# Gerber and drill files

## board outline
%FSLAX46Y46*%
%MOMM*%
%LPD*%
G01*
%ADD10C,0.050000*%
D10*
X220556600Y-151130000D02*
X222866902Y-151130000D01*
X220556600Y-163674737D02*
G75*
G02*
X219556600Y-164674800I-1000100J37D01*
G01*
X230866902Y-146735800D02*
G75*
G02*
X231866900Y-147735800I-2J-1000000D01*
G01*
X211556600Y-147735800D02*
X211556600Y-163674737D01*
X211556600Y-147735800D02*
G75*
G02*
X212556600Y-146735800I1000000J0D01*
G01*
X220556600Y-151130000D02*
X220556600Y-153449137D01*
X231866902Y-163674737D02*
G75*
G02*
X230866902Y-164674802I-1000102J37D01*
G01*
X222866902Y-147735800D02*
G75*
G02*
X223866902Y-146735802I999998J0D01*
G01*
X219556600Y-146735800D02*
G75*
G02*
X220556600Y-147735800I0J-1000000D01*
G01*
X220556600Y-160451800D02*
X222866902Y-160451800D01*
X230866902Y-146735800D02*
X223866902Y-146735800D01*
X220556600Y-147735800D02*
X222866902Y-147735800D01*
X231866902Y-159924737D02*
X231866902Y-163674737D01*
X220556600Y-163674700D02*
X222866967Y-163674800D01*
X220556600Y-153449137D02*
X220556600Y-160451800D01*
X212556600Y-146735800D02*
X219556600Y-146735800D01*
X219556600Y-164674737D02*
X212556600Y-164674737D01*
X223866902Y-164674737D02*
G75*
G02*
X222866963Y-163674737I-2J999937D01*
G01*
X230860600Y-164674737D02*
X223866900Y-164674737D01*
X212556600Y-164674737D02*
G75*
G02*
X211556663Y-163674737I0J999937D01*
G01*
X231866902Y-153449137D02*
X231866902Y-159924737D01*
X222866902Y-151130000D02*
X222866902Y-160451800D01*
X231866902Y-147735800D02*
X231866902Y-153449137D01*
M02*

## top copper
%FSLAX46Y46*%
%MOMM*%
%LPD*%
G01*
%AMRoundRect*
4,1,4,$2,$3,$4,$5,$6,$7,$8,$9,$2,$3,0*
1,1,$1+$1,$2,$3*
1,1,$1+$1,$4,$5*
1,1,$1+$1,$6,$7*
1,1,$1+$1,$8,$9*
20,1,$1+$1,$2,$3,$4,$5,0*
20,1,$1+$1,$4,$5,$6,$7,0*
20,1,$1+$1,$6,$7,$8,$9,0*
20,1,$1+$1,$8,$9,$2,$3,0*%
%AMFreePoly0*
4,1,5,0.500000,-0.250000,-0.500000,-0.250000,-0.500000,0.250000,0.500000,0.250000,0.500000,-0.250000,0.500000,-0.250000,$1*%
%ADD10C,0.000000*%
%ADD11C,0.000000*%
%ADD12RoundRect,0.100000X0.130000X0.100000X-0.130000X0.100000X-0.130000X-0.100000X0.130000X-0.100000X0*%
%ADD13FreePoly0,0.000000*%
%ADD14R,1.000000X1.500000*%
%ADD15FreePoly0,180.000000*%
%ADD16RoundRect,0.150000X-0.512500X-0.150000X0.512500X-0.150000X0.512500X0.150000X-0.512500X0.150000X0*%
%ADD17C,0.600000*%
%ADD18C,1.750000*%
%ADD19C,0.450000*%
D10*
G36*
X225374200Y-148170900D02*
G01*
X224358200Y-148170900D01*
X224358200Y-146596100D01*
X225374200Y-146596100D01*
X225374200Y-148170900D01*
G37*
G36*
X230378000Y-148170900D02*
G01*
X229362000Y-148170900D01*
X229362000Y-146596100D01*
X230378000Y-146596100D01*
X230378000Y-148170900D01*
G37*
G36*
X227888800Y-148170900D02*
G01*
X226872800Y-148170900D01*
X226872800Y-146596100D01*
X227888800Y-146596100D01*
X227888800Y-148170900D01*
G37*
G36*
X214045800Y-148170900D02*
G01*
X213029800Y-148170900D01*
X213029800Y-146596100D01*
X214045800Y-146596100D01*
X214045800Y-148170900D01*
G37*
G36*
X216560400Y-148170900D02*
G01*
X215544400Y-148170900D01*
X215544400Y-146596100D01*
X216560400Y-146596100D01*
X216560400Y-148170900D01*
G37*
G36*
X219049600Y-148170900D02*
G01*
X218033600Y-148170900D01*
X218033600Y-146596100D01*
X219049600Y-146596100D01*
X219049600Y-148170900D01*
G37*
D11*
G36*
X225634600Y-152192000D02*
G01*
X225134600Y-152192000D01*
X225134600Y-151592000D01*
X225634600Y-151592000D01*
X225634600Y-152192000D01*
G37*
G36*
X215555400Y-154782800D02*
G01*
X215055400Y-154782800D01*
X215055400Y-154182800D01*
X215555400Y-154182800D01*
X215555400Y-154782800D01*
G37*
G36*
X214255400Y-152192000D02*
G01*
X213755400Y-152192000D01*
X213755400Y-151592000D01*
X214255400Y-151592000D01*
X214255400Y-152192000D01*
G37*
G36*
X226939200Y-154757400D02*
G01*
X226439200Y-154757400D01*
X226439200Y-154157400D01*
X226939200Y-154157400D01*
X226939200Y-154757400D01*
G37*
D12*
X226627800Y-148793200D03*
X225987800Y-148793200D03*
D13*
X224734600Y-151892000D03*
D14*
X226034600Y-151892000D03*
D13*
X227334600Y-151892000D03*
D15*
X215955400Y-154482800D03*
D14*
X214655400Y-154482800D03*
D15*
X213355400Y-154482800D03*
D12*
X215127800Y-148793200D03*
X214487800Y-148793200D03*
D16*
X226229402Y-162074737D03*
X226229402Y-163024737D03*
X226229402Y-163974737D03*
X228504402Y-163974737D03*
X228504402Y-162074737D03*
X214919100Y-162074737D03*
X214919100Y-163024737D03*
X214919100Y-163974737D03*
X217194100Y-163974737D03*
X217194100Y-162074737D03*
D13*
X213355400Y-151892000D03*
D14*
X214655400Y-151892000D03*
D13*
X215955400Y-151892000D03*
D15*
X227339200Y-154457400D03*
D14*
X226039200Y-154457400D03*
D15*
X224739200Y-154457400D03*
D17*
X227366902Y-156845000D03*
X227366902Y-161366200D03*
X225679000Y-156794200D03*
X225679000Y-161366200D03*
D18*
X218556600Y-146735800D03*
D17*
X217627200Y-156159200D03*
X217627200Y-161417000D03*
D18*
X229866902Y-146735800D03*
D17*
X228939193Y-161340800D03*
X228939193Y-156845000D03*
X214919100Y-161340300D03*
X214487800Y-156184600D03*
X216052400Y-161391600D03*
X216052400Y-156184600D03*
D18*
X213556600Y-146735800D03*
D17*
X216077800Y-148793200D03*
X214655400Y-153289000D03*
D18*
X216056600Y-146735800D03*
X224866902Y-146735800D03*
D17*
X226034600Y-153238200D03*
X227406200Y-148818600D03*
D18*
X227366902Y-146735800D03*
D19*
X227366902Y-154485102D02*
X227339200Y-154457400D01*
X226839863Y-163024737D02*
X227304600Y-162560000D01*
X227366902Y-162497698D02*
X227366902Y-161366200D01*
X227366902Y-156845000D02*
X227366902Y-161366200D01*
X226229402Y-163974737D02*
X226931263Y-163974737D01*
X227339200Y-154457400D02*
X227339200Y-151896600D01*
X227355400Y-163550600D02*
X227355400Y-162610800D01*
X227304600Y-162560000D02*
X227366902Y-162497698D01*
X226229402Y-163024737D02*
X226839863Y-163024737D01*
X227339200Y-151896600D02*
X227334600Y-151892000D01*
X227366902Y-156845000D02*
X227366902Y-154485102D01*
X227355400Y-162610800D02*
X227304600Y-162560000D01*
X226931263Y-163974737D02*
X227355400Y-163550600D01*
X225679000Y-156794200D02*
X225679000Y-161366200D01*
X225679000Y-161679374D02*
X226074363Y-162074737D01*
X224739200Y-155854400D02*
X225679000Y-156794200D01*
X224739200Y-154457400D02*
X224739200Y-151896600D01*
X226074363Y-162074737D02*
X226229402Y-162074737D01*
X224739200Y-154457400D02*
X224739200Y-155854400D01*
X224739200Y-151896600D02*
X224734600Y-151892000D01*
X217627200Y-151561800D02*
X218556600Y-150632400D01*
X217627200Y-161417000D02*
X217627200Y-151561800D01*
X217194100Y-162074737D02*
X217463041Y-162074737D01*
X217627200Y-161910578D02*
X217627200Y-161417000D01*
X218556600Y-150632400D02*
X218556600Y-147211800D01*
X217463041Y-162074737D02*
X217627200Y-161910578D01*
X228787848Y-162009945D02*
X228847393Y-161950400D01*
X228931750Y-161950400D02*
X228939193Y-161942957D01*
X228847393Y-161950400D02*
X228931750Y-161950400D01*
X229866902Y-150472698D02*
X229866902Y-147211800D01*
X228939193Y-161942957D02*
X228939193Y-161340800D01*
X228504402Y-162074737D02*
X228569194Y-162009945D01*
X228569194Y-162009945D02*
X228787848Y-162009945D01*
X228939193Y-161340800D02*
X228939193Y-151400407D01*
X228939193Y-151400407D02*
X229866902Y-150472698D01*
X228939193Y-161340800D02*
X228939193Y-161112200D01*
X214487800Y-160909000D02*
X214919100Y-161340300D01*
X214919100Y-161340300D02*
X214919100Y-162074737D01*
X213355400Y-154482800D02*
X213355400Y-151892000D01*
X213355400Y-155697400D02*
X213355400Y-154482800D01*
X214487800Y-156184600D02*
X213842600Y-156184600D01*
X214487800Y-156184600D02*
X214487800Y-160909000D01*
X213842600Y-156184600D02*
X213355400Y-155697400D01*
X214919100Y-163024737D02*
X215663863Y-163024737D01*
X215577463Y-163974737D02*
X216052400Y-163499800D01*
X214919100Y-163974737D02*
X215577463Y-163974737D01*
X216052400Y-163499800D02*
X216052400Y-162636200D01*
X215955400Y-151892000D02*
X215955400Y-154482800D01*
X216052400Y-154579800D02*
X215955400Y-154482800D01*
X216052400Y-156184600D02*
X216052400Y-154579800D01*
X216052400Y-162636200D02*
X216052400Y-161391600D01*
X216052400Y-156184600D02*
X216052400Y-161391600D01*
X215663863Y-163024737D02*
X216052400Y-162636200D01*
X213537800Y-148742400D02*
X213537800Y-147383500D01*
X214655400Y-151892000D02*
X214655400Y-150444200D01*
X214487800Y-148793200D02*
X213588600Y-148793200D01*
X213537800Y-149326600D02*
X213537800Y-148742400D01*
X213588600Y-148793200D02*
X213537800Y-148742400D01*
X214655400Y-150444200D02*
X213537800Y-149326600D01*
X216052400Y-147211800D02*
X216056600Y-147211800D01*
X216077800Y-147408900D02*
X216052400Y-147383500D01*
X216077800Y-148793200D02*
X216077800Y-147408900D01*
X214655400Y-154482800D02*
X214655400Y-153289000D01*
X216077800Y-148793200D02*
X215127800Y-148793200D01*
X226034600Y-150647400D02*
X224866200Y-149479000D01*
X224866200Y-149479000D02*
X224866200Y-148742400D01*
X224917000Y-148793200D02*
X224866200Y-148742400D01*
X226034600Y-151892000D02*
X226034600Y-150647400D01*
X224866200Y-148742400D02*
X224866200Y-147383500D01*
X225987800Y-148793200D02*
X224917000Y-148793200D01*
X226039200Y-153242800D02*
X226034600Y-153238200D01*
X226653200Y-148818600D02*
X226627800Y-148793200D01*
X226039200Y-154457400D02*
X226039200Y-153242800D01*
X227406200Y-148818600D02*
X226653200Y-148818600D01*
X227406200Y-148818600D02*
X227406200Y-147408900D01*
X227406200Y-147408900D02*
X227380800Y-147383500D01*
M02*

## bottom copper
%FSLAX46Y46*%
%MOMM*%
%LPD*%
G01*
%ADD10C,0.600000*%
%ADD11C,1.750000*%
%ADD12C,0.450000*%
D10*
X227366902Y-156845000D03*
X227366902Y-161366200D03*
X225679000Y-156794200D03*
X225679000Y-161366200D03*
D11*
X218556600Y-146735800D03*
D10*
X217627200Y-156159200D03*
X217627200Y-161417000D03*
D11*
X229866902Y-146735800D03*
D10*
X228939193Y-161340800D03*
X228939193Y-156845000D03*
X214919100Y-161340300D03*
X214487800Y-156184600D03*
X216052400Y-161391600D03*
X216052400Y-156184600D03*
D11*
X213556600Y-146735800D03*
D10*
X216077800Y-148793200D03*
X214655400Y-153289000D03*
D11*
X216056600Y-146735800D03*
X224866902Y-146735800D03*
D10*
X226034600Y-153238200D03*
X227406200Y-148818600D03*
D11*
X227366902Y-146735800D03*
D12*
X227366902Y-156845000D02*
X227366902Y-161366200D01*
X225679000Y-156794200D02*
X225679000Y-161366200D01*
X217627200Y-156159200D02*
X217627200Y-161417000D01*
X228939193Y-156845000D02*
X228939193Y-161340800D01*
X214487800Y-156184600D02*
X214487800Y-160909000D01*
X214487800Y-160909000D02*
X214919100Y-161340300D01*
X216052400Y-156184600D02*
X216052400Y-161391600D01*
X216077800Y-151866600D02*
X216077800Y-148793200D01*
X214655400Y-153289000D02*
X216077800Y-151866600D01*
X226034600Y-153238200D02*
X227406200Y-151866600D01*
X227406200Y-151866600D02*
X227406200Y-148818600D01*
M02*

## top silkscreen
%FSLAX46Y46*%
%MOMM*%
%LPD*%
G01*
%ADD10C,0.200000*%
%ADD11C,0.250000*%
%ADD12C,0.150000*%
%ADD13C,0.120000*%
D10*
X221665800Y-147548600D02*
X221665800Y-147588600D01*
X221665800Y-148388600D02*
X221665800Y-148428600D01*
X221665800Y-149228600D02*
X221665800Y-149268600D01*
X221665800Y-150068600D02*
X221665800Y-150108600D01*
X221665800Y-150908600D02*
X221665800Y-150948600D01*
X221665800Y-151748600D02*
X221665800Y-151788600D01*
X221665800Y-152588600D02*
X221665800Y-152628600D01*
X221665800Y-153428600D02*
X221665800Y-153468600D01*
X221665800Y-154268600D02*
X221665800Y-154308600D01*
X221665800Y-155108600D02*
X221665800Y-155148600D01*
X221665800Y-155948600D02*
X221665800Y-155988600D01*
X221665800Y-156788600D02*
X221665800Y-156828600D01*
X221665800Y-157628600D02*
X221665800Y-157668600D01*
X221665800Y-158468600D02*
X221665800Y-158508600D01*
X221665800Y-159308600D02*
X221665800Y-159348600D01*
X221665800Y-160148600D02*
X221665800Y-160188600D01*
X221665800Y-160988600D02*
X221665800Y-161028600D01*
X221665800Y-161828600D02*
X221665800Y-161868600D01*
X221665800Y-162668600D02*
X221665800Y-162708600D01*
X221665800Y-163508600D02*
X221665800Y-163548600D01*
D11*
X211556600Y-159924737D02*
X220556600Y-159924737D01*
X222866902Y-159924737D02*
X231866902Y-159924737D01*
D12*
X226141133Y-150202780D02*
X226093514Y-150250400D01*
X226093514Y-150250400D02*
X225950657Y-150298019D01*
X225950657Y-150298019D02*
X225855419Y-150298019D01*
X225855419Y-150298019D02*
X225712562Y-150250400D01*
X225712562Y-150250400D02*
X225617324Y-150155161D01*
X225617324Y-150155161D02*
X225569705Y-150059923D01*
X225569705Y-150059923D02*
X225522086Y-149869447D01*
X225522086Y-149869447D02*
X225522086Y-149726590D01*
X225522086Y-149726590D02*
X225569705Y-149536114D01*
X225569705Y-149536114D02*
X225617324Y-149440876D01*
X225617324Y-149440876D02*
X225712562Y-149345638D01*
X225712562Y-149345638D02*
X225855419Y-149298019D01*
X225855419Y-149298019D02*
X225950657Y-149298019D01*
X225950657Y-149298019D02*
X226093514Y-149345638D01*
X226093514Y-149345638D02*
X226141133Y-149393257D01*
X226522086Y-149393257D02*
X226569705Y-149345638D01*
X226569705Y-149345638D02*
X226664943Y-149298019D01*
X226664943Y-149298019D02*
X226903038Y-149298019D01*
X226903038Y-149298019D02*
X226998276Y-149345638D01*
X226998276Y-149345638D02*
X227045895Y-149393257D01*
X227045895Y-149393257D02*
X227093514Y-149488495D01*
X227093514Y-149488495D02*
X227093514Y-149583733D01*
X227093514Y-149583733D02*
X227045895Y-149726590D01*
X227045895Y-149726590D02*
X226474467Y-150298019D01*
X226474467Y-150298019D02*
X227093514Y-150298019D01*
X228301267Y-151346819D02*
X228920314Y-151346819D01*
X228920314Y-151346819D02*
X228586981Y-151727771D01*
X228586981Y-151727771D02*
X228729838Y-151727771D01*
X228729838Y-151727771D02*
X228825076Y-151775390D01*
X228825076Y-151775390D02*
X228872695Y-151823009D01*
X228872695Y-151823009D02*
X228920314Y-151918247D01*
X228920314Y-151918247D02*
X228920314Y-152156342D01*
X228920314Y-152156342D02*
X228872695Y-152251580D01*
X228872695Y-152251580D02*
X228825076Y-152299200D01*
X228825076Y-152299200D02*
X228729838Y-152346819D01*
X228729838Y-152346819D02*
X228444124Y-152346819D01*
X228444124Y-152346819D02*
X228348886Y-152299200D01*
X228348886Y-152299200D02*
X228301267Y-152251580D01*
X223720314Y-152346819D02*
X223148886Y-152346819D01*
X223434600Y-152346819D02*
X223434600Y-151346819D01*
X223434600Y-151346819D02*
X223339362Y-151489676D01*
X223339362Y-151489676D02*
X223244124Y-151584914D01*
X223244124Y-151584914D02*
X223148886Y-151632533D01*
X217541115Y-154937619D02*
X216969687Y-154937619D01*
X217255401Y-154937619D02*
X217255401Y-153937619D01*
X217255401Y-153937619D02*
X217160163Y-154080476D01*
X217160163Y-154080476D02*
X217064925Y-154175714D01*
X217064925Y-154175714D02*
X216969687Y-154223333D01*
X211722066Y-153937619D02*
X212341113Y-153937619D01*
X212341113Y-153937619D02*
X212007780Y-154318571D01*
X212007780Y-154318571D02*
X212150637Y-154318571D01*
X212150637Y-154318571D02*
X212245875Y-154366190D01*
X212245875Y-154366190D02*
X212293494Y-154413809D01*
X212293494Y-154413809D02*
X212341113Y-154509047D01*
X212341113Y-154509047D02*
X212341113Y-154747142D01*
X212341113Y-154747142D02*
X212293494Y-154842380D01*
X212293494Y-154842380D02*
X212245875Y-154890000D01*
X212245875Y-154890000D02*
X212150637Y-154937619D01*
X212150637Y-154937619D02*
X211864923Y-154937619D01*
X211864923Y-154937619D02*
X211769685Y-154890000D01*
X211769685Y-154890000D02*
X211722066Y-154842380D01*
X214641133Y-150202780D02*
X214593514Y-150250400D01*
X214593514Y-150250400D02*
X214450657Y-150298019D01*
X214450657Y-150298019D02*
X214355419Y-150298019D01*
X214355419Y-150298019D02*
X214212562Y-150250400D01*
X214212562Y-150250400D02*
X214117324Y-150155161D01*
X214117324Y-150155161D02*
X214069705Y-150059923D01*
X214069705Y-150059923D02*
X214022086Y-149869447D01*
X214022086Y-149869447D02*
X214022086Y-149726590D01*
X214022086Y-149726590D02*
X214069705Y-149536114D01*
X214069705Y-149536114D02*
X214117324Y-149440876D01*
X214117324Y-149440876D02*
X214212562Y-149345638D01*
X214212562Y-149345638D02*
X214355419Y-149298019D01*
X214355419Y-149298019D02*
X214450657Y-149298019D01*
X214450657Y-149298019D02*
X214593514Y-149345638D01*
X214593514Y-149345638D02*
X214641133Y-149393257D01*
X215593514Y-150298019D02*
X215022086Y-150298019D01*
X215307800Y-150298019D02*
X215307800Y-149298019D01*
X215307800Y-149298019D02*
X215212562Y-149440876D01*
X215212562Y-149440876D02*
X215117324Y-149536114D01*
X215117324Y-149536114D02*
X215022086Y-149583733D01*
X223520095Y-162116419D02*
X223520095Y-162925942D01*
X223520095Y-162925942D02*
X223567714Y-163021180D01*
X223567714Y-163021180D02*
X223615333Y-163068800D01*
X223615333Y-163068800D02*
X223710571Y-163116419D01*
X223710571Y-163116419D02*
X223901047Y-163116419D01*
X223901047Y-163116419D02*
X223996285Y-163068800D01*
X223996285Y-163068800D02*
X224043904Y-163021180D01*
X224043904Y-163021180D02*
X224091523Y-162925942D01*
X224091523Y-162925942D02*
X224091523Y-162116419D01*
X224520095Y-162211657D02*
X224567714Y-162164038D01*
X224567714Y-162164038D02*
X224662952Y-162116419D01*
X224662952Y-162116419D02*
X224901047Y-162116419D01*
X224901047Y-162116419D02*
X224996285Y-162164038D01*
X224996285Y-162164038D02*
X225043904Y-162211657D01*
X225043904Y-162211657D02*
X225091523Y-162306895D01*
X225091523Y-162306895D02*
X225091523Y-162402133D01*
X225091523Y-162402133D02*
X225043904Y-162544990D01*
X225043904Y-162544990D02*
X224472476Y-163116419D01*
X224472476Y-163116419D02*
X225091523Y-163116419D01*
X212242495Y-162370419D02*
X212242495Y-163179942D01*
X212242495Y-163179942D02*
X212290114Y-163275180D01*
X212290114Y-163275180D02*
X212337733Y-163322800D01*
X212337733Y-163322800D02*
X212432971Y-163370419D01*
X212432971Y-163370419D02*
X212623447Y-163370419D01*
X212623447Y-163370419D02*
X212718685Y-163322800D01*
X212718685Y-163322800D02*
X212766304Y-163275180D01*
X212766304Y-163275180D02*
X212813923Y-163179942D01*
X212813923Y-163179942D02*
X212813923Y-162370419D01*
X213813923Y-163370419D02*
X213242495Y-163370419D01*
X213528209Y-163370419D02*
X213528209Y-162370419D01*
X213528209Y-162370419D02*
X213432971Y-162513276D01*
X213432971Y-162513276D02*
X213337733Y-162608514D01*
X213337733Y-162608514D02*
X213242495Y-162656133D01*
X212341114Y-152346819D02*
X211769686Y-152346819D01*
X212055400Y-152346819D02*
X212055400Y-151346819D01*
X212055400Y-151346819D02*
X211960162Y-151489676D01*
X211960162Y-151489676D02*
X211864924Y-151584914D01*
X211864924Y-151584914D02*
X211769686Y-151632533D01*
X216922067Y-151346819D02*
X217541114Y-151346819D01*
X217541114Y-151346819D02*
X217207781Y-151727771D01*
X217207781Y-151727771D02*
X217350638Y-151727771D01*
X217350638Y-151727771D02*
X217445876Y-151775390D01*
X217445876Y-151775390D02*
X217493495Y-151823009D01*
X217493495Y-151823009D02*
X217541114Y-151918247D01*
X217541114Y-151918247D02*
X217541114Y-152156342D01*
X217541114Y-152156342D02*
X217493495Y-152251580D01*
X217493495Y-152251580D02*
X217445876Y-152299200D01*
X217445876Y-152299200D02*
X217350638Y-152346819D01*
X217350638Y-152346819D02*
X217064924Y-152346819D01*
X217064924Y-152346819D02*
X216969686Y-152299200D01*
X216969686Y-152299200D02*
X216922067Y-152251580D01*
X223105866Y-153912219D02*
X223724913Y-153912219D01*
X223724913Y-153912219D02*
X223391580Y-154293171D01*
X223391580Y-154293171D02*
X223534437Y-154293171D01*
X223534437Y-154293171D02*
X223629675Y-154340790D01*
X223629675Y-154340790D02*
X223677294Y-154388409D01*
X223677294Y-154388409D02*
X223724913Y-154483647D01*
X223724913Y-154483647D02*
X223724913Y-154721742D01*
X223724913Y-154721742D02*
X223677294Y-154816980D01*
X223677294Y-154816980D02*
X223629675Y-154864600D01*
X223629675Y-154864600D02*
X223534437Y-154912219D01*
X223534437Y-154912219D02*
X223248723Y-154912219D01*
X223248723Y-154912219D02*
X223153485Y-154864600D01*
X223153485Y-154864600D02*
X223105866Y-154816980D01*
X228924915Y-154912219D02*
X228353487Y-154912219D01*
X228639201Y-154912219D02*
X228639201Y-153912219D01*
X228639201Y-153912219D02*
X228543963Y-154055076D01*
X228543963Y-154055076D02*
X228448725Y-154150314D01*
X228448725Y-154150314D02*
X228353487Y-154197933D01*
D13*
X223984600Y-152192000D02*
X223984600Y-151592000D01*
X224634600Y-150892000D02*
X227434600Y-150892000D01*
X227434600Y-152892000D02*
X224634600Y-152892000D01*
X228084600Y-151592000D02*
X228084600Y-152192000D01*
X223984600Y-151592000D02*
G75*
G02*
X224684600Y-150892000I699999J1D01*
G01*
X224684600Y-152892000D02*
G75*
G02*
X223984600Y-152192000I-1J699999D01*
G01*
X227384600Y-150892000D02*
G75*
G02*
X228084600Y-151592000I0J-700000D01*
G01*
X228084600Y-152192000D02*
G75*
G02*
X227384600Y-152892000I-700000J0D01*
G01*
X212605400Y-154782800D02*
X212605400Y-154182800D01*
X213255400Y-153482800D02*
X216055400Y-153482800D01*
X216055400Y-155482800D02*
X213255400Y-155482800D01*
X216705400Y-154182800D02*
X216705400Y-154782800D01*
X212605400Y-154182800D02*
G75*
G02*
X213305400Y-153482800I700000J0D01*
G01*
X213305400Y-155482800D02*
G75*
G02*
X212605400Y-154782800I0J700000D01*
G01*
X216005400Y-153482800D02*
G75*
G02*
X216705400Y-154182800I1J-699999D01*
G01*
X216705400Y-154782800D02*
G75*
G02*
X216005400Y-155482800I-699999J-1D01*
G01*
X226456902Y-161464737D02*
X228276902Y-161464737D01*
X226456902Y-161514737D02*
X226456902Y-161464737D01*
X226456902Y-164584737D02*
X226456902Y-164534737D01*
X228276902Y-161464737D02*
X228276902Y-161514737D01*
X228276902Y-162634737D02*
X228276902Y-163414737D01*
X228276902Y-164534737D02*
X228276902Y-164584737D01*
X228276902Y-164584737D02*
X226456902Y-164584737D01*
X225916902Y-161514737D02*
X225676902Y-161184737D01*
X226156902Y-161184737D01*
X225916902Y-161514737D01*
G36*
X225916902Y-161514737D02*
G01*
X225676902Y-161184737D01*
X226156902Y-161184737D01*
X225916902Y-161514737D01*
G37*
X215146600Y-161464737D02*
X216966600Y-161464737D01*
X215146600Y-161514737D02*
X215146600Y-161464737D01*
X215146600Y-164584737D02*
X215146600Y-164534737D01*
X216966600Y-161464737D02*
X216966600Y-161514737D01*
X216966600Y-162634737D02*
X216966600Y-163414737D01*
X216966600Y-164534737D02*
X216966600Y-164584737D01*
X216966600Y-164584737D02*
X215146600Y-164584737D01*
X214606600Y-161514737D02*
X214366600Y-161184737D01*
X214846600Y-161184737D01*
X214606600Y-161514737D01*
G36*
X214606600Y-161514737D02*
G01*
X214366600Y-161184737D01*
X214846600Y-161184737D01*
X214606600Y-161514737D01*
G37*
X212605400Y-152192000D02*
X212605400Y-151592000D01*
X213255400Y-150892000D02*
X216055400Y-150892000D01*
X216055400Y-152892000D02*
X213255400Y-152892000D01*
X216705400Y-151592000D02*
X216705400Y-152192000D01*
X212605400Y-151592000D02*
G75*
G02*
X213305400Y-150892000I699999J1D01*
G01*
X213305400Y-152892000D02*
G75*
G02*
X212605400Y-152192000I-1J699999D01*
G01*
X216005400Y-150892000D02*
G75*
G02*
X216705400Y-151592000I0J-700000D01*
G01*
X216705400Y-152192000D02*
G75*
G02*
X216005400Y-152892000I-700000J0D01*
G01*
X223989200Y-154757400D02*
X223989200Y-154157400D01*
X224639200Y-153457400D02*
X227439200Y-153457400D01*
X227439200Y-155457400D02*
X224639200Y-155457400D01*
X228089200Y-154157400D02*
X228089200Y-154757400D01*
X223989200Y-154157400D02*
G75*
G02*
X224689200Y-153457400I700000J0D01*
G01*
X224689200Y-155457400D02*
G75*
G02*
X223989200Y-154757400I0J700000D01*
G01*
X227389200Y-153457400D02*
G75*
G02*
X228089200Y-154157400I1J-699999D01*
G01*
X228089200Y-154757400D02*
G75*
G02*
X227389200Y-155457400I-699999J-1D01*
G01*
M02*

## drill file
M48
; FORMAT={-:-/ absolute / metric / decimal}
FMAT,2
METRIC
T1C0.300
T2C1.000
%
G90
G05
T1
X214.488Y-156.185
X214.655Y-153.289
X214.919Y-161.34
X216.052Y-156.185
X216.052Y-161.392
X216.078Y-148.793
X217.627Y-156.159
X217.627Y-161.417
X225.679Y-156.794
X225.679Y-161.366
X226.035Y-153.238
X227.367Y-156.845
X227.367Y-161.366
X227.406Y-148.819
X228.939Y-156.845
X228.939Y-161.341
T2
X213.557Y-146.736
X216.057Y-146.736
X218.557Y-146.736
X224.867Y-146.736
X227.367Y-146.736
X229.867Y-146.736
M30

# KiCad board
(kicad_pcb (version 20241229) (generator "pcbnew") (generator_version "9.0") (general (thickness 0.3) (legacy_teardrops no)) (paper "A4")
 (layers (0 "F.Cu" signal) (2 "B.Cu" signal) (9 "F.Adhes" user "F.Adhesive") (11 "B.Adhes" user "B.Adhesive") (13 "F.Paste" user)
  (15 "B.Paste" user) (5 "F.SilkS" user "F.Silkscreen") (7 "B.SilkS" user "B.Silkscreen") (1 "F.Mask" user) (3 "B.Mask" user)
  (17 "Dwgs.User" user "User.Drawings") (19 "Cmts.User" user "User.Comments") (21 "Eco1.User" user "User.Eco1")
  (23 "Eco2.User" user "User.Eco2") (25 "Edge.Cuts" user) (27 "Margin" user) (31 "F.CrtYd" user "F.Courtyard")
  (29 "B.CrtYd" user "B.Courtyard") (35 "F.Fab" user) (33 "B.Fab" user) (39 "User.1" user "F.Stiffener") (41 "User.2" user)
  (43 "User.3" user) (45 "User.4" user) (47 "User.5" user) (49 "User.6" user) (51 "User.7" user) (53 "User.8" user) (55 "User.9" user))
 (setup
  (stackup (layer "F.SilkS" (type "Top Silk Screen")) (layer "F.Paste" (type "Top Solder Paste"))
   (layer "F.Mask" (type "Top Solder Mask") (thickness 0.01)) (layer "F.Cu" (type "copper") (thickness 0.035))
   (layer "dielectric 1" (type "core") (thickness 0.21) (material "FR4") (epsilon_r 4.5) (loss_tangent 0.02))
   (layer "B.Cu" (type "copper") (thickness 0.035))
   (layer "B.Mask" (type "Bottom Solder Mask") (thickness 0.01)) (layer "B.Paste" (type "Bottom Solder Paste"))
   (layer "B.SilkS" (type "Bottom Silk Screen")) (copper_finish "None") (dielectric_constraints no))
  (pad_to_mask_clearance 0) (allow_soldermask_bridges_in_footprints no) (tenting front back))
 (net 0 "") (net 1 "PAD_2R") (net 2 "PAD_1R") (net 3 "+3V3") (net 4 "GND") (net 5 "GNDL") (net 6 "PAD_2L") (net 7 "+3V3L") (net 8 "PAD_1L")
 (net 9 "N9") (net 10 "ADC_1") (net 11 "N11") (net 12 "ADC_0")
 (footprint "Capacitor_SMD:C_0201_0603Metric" (layer "F.Cu") (at 226.3078 148.7932 180)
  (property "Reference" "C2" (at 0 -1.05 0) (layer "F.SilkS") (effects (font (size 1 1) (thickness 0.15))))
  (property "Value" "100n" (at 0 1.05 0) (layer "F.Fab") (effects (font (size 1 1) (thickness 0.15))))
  (pad "" smd roundrect (at -0.345 0 180) (size 0.318 0.36) (layers "F.Paste") (roundrect_rratio 0.25))
  (pad "" smd roundrect (at 0.345 0 180) (size 0.318 0.36) (layers "F.Paste") (roundrect_rratio 0.25))
  (pad "1" smd roundrect (at -0.32 0 180) (size 0.46 0.4) (layers "F.Cu" "F.Mask") (roundrect_rratio 0.25) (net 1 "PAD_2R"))
  (pad "2" smd roundrect (at 0.32 0 180) (size 0.46 0.4) (layers "F.Cu" "F.Mask") (roundrect_rratio 0.25) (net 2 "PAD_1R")))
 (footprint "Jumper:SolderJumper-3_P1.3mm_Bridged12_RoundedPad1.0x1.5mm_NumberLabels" (layer "F.Cu") (at 226.0346 151.892)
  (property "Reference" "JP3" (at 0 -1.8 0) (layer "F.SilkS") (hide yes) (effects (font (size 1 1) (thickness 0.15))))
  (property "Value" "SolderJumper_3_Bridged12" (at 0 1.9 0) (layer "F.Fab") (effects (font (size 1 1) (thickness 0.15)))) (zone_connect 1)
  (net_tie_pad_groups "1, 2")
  (fp_poly (pts (xy -0.9 -0.3) (xy -0.4 -0.3) (xy -0.4 0.3) (xy -0.9 0.3)) (stroke (width 0) (type solid)) (fill yes) (layer "F.Cu"))
  (fp_line (start -2.05 0.3) (end -2.05 -0.3) (stroke (width 0.12) (type solid)) (layer "F.SilkS"))
  (fp_line (start -1.4 -1) (end 1.4 -1) (stroke (width 0.12) (type solid)) (layer "F.SilkS"))
  (fp_line (start 1.4 1) (end -1.4 1) (stroke (width 0.12) (type solid)) (layer "F.SilkS"))
  (fp_line (start 2.05 -0.3) (end 2.05 0.3) (stroke (width 0.12) (type solid)) (layer "F.SilkS"))
  (fp_arc (start -2.05 -0.3) (mid -1.844975 -0.794975) (end -1.35 -1) (stroke (width 0.12) (type solid)) (layer "F.SilkS"))
  (fp_arc (start -1.35 1) (mid -1.844975 0.794975) (end -2.05 0.3) (stroke (width 0.12) (type solid)) (layer "F.SilkS"))
  (fp_arc (start 1.35 -1) (mid 1.844975 -0.794975) (end 2.05 -0.3) (stroke (width 0.12) (type solid)) (layer "F.SilkS"))
  (fp_arc (start 2.05 0.3) (mid 1.844975 0.794975) (end 1.35 1) (stroke (width 0.12) (type solid)) (layer "F.SilkS"))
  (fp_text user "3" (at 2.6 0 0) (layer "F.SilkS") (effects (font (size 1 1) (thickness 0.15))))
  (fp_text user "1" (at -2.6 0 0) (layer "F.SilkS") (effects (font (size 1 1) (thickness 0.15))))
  (pad "1" smd custom (at -1.3 0) (size 1 0.5) (layers "F.Cu" "F.Mask") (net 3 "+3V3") (zone_connect 2) (thermal_bridge_angle 45)
   (options (clearance outline) (anchor rect)) (primitives))
  (pad "2" smd rect (at 0 0) (size 1 1.5) (layers "F.Cu" "F.Mask") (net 2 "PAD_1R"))
  (pad "3" smd custom (at 1.3 0) (size 1 0.5) (layers "F.Cu" "F.Mask") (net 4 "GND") (zone_connect 2) (thermal_bridge_angle 45)
   (options (clearance outline) (anchor rect)) (primitives)))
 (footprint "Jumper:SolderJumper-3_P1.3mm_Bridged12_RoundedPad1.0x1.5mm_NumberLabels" (layer "F.Cu") (at 214.6554 154.4828 180)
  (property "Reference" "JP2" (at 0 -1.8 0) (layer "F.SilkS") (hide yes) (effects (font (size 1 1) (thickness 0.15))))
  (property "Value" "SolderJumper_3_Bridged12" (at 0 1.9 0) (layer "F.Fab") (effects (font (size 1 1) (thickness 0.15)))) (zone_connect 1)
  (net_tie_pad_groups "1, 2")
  (fp_poly (pts (xy -0.9 -0.3) (xy -0.4 -0.3) (xy -0.4 0.3) (xy -0.9 0.3)) (stroke (width 0) (type solid)) (fill yes) (layer "F.Cu"))
  (fp_line (start 2.05 -0.3) (end 2.05 0.3) (stroke (width 0.12) (type solid)) (layer "F.SilkS"))
  (fp_line (start 1.4 1) (end -1.4 1) (stroke (width 0.12) (type solid)) (layer "F.SilkS"))
  (fp_line (start -1.4 -1) (end 1.4 -1) (stroke (width 0.12) (type solid)) (layer "F.SilkS"))
  (fp_line (start -2.05 0.3) (end -2.05 -0.3) (stroke (width 0.12) (type solid)) (layer "F.SilkS"))
  (fp_arc (start 2.05 0.3) (mid 1.844975 0.794975) (end 1.35 1) (stroke (width 0.12) (type solid)) (layer "F.SilkS"))
  (fp_arc (start 1.35 -1) (mid 1.844975 -0.794975) (end 2.05 -0.3) (stroke (width 0.12) (type solid)) (layer "F.SilkS"))
  (fp_arc (start -1.35 1) (mid -1.844975 0.794975) (end -2.05 0.3) (stroke (width 0.12) (type solid)) (layer "F.SilkS"))
  (fp_arc (start -2.05 -0.3) (mid -1.844975 -0.794975) (end -1.35 -1) (stroke (width 0.12) (type solid)) (layer "F.SilkS"))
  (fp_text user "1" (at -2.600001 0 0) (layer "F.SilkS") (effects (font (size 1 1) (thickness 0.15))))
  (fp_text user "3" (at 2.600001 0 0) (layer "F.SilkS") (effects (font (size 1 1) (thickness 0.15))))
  (pad "1" smd custom (at -1.3 0 180) (size 1 0.5) (layers "F.Cu" "F.Mask") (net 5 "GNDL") (zone_connect 2) (thermal_bridge_angle 45)
   (options (clearance outline) (anchor rect)) (primitives))
  (pad "2" smd rect (at 0 0 180) (size 1 1.5) (layers "F.Cu" "F.Mask") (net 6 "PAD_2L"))
  (pad "3" smd custom (at 1.3 0 180) (size 1 0.5) (layers "F.Cu" "F.Mask") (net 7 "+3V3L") (zone_connect 2) (thermal_bridge_angle 45)
   (options (clearance outline) (anchor rect)) (primitives)))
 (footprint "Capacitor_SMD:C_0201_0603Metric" (layer "F.Cu") (at 214.8078 148.7932 180)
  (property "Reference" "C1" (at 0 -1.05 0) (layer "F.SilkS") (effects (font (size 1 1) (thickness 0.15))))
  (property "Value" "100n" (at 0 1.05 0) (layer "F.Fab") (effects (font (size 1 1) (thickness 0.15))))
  (pad "" smd roundrect (at -0.345 0 180) (size 0.318 0.36) (layers "F.Paste") (roundrect_rratio 0.25))
  (pad "" smd roundrect (at 0.345 0 180) (size 0.318 0.36) (layers "F.Paste") (roundrect_rratio 0.25))
  (pad "1" smd roundrect (at -0.32 0 180) (size 0.46 0.4) (layers "F.Cu" "F.Mask") (roundrect_rratio 0.25) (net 6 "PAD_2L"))
  (pad "2" smd roundrect (at 0.32 0 180) (size 0.46 0.4) (layers "F.Cu" "F.Mask") (roundrect_rratio 0.25) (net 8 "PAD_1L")))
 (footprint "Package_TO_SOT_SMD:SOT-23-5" (layer "F.Cu") (at 227.366902 163.024737)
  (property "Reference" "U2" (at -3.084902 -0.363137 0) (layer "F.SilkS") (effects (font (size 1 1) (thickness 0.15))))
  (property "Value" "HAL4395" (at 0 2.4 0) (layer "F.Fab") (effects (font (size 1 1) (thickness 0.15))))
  (fp_line (start -0.91 -1.56) (end 0.91 -1.56) (stroke (width 0.12) (type solid)) (layer "F.SilkS"))
  (fp_line (start -0.91 -1.51) (end -0.91 -1.56) (stroke (width 0.12) (type solid)) (layer "F.SilkS"))
  (fp_line (start -0.91 1.56) (end -0.91 1.51) (stroke (width 0.12) (type solid)) (layer "F.SilkS"))
  (fp_line (start 0.91 -1.56) (end 0.91 -1.51) (stroke (width 0.12) (type solid)) (layer "F.SilkS"))
  (fp_line (start 0.91 -0.39) (end 0.91 0.39) (stroke (width 0.12) (type solid)) (layer "F.SilkS"))
  (fp_line (start 0.91 1.51) (end 0.91 1.56) (stroke (width 0.12) (type solid)) (layer "F.SilkS"))
  (fp_line (start 0.91 1.56) (end -0.91 1.56) (stroke (width 0.12) (type solid)) (layer "F.SilkS"))
  (fp_poly (pts (xy -1.45 -1.51) (xy -1.69 -1.84) (xy -1.21 -1.84)) (stroke (width 0.12) (type solid)) (fill yes) (layer "F.SilkS"))
  (pad "1" smd roundrect (at -1.1375 -0.95) (size 1.325 0.6) (layers "F.Cu" "F.Mask" "F.Paste") (roundrect_rratio 0.25) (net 3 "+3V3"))
  (pad "2" smd roundrect (at -1.1375 0) (size 1.325 0.6) (layers "F.Cu" "F.Mask" "F.Paste") (roundrect_rratio 0.25) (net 4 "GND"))
  (pad "3" smd roundrect (at -1.1375 0.95) (size 1.325 0.6) (layers "F.Cu" "F.Mask" "F.Paste") (roundrect_rratio 0.25) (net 4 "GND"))
  (pad "4" smd roundrect (at 1.1375 0.95) (size 1.325 0.6) (layers "F.Cu" "F.Mask" "F.Paste") (roundrect_rratio 0.25) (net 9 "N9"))
  (pad "5" smd roundrect (at 1.1375 -0.95) (size 1.325 0.6) (layers "F.Cu" "F.Mask" "F.Paste") (roundrect_rratio 0.25) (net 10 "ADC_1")))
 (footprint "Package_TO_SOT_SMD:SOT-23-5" (layer "F.Cu") (at 216.0566 163.024737)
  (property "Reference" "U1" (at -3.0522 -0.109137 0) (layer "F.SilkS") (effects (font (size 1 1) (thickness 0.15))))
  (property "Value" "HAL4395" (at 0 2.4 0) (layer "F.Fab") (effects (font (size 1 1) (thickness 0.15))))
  (fp_line (start -0.91 -1.56) (end 0.91 -1.56) (stroke (width 0.12) (type solid)) (layer "F.SilkS"))
  (fp_line (start -0.91 -1.51) (end -0.91 -1.56) (stroke (width 0.12) (type solid)) (layer "F.SilkS"))
  (fp_line (start -0.91 1.56) (end -0.91 1.51) (stroke (width 0.12) (type solid)) (layer "F.SilkS"))
  (fp_line (start 0.91 -1.56) (end 0.91 -1.51) (stroke (width 0.12) (type solid)) (layer "F.SilkS"))
  (fp_line (start 0.91 -0.39) (end 0.91 0.39) (stroke (width 0.12) (type solid)) (layer "F.SilkS"))
  (fp_line (start 0.91 1.51) (end 0.91 1.56) (stroke (width 0.12) (type solid)) (layer "F.SilkS"))
  (fp_line (start 0.91 1.56) (end -0.91 1.56) (stroke (width 0.12) (type solid)) (layer "F.SilkS"))
  (fp_poly (pts (xy -1.45 -1.51) (xy -1.69 -1.84) (xy -1.21 -1.84)) (stroke (width 0.12) (type solid)) (fill yes) (layer "F.SilkS"))
  (pad "1" smd roundrect (at -1.1375 -0.95) (size 1.325 0.6) (layers "F.Cu" "F.Mask" "F.Paste") (roundrect_rratio 0.25) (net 7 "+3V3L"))
  (pad "2" smd roundrect (at -1.1375 0) (size 1.325 0.6) (layers "F.Cu" "F.Mask" "F.Paste") (roundrect_rratio 0.25) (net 5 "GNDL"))
  (pad "3" smd roundrect (at -1.1375 0.95) (size 1.325 0.6) (layers "F.Cu" "F.Mask" "F.Paste") (roundrect_rratio 0.25) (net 5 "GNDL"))
  (pad "4" smd roundrect (at 1.1375 0.95) (size 1.325 0.6) (layers "F.Cu" "F.Mask" "F.Paste") (roundrect_rratio 0.25) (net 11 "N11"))
  (pad "5" smd roundrect (at 1.1375 -0.95) (size 1.325 0.6) (layers "F.Cu" "F.Mask" "F.Paste") (roundrect_rratio 0.25) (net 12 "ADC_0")))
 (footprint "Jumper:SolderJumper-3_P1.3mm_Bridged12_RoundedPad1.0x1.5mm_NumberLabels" (layer "F.Cu") (at 214.6554 151.892)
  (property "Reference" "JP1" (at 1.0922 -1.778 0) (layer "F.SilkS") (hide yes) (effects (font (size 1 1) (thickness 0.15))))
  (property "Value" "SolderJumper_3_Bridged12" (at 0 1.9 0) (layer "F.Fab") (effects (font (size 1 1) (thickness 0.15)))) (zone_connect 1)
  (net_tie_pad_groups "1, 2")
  (fp_poly (pts (xy -0.9 -0.3) (xy -0.4 -0.3) (xy -0.4 0.3) (xy -0.9 0.3)) (stroke (width 0) (type solid)) (fill yes) (layer "F.Cu"))
  (fp_line (start -2.05 0.3) (end -2.05 -0.3) (stroke (width 0.12) (type solid)) (layer "F.SilkS"))
  (fp_line (start -1.4 -1) (end 1.4 -1) (stroke (width 0.12) (type solid)) (layer "F.SilkS"))
  (fp_line (start 1.4 1) (end -1.4 1) (stroke (width 0.12) (type solid)) (layer "F.SilkS"))
  (fp_line (start 2.05 -0.3) (end 2.05 0.3) (stroke (width 0.12) (type solid)) (layer "F.SilkS"))
  (fp_arc (start -2.05 -0.3) (mid -1.844975 -0.794975) (end -1.35 -1) (stroke (width 0.12) (type solid)) (layer "F.SilkS"))
  (fp_arc (start -1.35 1) (mid -1.844975 0.794975) (end -2.05 0.3) (stroke (width 0.12) (type solid)) (layer "F.SilkS"))
  (fp_arc (start 1.35 -1) (mid 1.844975 -0.794975) (end 2.05 -0.3) (stroke (width 0.12) (type solid)) (layer "F.SilkS"))
  (fp_arc (start 2.05 0.3) (mid 1.844975 0.794975) (end 1.35 1) (stroke (width 0.12) (type solid)) (layer "F.SilkS"))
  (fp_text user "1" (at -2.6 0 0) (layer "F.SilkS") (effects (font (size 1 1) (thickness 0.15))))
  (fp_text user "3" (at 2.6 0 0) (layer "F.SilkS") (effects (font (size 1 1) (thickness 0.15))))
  (pad "1" smd custom (at -1.3 0) (size 1 0.5) (layers "F.Cu" "F.Mask") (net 7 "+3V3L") (zone_connect 2) (thermal_bridge_angle 45)
   (options (clearance outline) (anchor rect)) (primitives))
  (pad "2" smd rect (at 0 0) (size 1 1.5) (layers "F.Cu" "F.Mask") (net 8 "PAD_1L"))
  (pad "3" smd custom (at 1.3 0) (size 1 0.5) (layers "F.Cu" "F.Mask") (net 5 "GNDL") (zone_connect 2) (thermal_bridge_angle 45)
   (options (clearance outline) (anchor rect)) (primitives)))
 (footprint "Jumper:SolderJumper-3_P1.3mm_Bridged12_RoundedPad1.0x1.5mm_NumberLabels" (layer "F.Cu") (at 226.0392 154.4574 180)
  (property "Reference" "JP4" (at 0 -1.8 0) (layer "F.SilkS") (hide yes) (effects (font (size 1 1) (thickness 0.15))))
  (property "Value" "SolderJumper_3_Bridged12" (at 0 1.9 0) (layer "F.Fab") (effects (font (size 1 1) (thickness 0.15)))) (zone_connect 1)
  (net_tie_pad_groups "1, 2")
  (fp_poly (pts (xy -0.9 -0.3) (xy -0.4 -0.3) (xy -0.4 0.3) (xy -0.9 0.3)) (stroke (width 0) (type solid)) (fill yes) (layer "F.Cu"))
  (fp_line (start 2.05 -0.3) (end 2.05 0.3) (stroke (width 0.12) (type solid)) (layer "F.SilkS"))
  (fp_line (start 1.4 1) (end -1.4 1) (stroke (width 0.12) (type solid)) (layer "F.SilkS"))
  (fp_line (start -1.4 -1) (end 1.4 -1) (stroke (width 0.12) (type solid)) (layer "F.SilkS"))
  (fp_line (start -2.05 0.3) (end -2.05 -0.3) (stroke (width 0.12) (type solid)) (layer "F.SilkS"))
  (fp_arc (start 2.05 0.3) (mid 1.844975 0.794975) (end 1.35 1) (stroke (width 0.12) (type solid)) (layer "F.SilkS"))
  (fp_arc (start 1.35 -1) (mid 1.844975 -0.794975) (end 2.05 -0.3) (stroke (width 0.12) (type solid)) (layer "F.SilkS"))
  (fp_arc (start -1.35 1) (mid -1.844975 0.794975) (end -2.05 0.3) (stroke (width 0.12) (type solid)) (layer "F.SilkS"))
  (fp_arc (start -2.05 -0.3) (mid -1.844975 -0.794975) (end -1.35 -1) (stroke (width 0.12) (type solid)) (layer "F.SilkS"))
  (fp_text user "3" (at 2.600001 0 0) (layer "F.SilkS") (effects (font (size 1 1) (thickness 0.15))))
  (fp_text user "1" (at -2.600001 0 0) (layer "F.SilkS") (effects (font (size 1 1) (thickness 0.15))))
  (pad "1" smd custom (at -1.3 0 180) (size 1 0.5) (layers "F.Cu" "F.Mask") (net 4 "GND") (zone_connect 2) (thermal_bridge_angle 45)
   (options (clearance outline) (anchor rect)) (primitives))
  (pad "2" smd rect (at 0 0 180) (size 1 1.5) (layers "F.Cu" "F.Mask") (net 1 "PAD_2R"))
  (pad "3" smd custom (at 1.3 0 180) (size 1 0.5) (layers "F.Cu" "F.Mask") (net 3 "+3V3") (zone_connect 2) (thermal_bridge_angle 45)
   (options (clearance outline) (anchor rect)) (primitives)))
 (gr_poly
  (pts (xy 224.3582 146.5961) (xy 225.3742 146.5961) (xy 225.3742 148.1709) (xy 224.3582 148.1709)) (stroke (width 0) (type solid))
  (fill yes) (layer "F.Cu") (net 2))
 (gr_poly
  (pts (xy 229.362 146.5961) (xy 230.378 146.5961) (xy 230.378 148.1709) (xy 229.362 148.1709)) (stroke (width 0) (type solid)) (fill yes)
  (layer "F.Cu") (net 10))
 (gr_poly
  (pts (xy 226.8728 146.5961) (xy 227.8888 146.5961) (xy 227.8888 148.1709) (xy 226.8728 148.1709)) (stroke (width 0) (type solid))
  (fill yes) (layer "F.Cu") (net 1))
 (gr_poly
  (pts (xy 213.0298 146.5961) (xy 214.0458 146.5961) (xy 214.0458 148.1709) (xy 213.0298 148.1709)) (stroke (width 0) (type solid))
  (fill yes) (layer "F.Cu") (net 8))
 (gr_poly
  (pts (xy 215.5444 146.5961) (xy 216.5604 146.5961) (xy 216.5604 148.1709) (xy 215.5444 148.1709)) (stroke (width 0) (type solid))
  (fill yes) (layer "F.Cu") (net 6))
 (gr_poly
  (pts (xy 218.0336 146.5961) (xy 219.0496 146.5961) (xy 219.0496 148.1709) (xy 218.0336 148.1709)) (stroke (width 0) (type solid))
  (fill yes) (layer "F.Cu") (net 12))
 (gr_line (start 221.6658 147.5486) (end 221.6658 164.0332) (stroke (width 0.2) (type dot)) (layer "F.SilkS"))
 (gr_line (start 211.5566 159.924737) (end 220.5566 159.924737) (stroke (width 0.25) (type solid)) (layer "F.SilkS"))
 (gr_line (start 222.866902 159.924737) (end 231.866902 159.924737) (stroke (width 0.25) (type solid)) (layer "F.SilkS"))
 (gr_line (start 220.5566 151.13) (end 222.866902 151.13) (stroke (width 0.05) (type default)) (layer "Edge.Cuts"))
 (gr_arc (start 220.5566 163.674737) (mid 220.263694 164.38182) (end 219.5566 164.674737) (stroke (width 0.05) (type default))
  (layer "Edge.Cuts"))
 (gr_arc (start 230.866902 146.7358) (mid 231.574009 147.028693) (end 231.866902 147.7358) (stroke (width 0.05) (type default))
  (layer "Edge.Cuts"))
 (gr_line (start 211.5566 147.7358) (end 211.5566 163.674737) (stroke (width 0.05) (type default)) (layer "Edge.Cuts"))
 (gr_arc (start 211.5566 147.7358) (mid 211.849493 147.028693) (end 212.5566 146.7358) (stroke (width 0.05) (type default))
  (layer "Edge.Cuts"))
 (gr_line (start 220.5566 151.13) (end 220.5566 153.449137) (stroke (width 0.05) (type default)) (layer "Edge.Cuts"))
 (gr_arc (start 231.866902 163.674737) (mid 231.573996 164.38182) (end 230.866902 164.674737) (stroke (width 0.05) (type default))
  (layer "Edge.Cuts"))
 (gr_arc (start 222.866902 147.7358) (mid 223.159795 147.028693) (end 223.866902 146.7358) (stroke (width 0.05) (type default))
  (layer "Edge.Cuts"))
 (gr_arc (start 219.5566 146.7358) (mid 220.263707 147.028693) (end 220.5566 147.7358) (stroke (width 0.05) (type default))
  (layer "Edge.Cuts"))
 (gr_line (start 220.5566 160.4518) (end 222.866902 160.4518) (stroke (width 0.05) (type default)) (layer "Edge.Cuts"))
 (gr_line (start 230.866902 146.7358) (end 223.866902 146.7358) (stroke (width 0.05) (type default)) (layer "Edge.Cuts"))
 (gr_line (start 220.5566 147.7358) (end 222.866902 147.7358) (stroke (width 0.05) (type default)) (layer "Edge.Cuts"))
 (gr_line (start 231.866902 159.924737) (end 231.866902 163.674737) (stroke (width 0.05) (type default)) (layer "Edge.Cuts"))
 (gr_line (start 220.5566 163.6747) (end 222.866967 163.6748) (stroke (width 0.05) (type default)) (layer "Edge.Cuts"))
 (gr_line (start 220.5566 153.449137) (end 220.5566 160.4518) (stroke (width 0.05) (type default)) (layer "Edge.Cuts"))
 (gr_line (start 212.5566 146.7358) (end 219.5566 146.7358) (stroke (width 0.05) (type default)) (layer "Edge.Cuts"))
 (gr_line (start 219.5566 164.674737) (end 212.5566 164.674737) (stroke (width 0.05) (type default)) (layer "Edge.Cuts"))
 (gr_arc (start 223.866902 164.674737) (mid 223.159782 164.381846) (end 222.866902 163.674737) (stroke (width 0.05) (type default))
  (layer "Edge.Cuts"))
 (gr_line (start 230.8606 164.674737) (end 223.8669 164.674737) (stroke (width 0.05) (type default)) (layer "Edge.Cuts"))
 (gr_arc (start 212.5566 164.674737) (mid 211.84948 164.381846) (end 211.5566 163.674737) (stroke (width 0.05) (type default))
  (layer "Edge.Cuts"))
 (gr_line (start 231.866902 153.449137) (end 231.866902 159.924737) (stroke (width 0.05) (type default)) (layer "Edge.Cuts"))
 (gr_line (start 222.866902 151.13) (end 222.866902 160.4518) (stroke (width 0.05) (type default)) (layer "Edge.Cuts"))
 (gr_line (start 231.866902 147.7358) (end 231.866902 153.449137) (stroke (width 0.05) (type default)) (layer "Edge.Cuts"))
 (segment (start 227.366902 154.485102) (end 227.3392 154.4574) (width 0.45) (layer "F.Cu") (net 4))
 (segment (start 226.839863 163.024737) (end 227.3046 162.56) (width 0.45) (layer "F.Cu") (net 4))
 (segment (start 227.366902 162.497698) (end 227.366902 161.3662) (width 0.45) (layer "F.Cu") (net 4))
 (segment (start 227.366902 156.845) (end 227.366902 161.3662) (width 0.45) (layer "F.Cu") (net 4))
 (segment (start 226.229402 163.974737) (end 226.931263 163.974737) (width 0.45) (layer "F.Cu") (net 4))
 (segment (start 227.3392 154.4574) (end 227.3392 151.8966) (width 0.45) (layer "F.Cu") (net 4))
 (segment (start 227.3554 163.5506) (end 227.3554 162.6108) (width 0.45) (layer "F.Cu") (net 4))
 (segment (start 227.3046 162.56) (end 227.366902 162.497698) (width 0.45) (layer "F.Cu") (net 4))
 (segment (start 226.229402 163.024737) (end 226.839863 163.024737) (width 0.45) (layer "F.Cu") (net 4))
 (segment (start 227.3392 151.8966) (end 227.3346 151.892) (width 0.45) (layer "F.Cu") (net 4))
 (segment (start 227.366902 156.845) (end 227.366902 154.485102) (width 0.45) (layer "F.Cu") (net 4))
 (segment (start 227.3554 162.6108) (end 227.3046 162.56) (width 0.45) (layer "F.Cu") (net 4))
 (segment (start 226.931263 163.974737) (end 227.3554 163.5506) (width 0.45) (layer "F.Cu") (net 4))
 (via (at 227.366902 156.845) (size 0.6) (drill 0.3) (layers "F.Cu" "B.Cu") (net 4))
 (via (at 227.366902 161.3662) (size 0.6) (drill 0.3) (layers "F.Cu" "B.Cu") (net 4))
 (segment (start 227.366902 156.845) (end 227.366902 161.3662) (width 0.45) (layer "B.Cu") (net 4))
 (segment (start 225.679 156.7942) (end 225.679 161.3662) (width 0.45) (layer "F.Cu") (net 3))
 (segment (start 225.679 161.679374) (end 226.074363 162.074737) (width 0.45) (layer "F.Cu") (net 3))
 (segment (start 224.7392 155.8544) (end 225.679 156.7942) (width 0.45) (layer "F.Cu") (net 3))
 (segment (start 224.7392 154.4574) (end 224.7392 151.8966) (width 0.45) (layer "F.Cu") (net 3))
 (segment (start 226.074363 162.074737) (end 226.229402 162.074737) (width 0.45) (layer "F.Cu") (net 3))
 (segment (start 224.7392 154.4574) (end 224.7392 155.8544) (width 0.45) (layer "F.Cu") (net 3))
 (segment (start 224.7392 151.8966) (end 224.7346 151.892) (width 0.45) (layer "F.Cu") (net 3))
 (via (at 225.679 156.7942) (size 0.6) (drill 0.3) (layers "F.Cu" "B.Cu") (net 3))
 (via (at 225.679 161.3662) (size 0.6) (drill 0.3) (layers "F.Cu" "B.Cu") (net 3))
 (segment (start 225.679 156.7942) (end 225.679 161.3662) (width 0.45) (layer "B.Cu") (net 3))
 (segment (start 217.6272 151.5618) (end 218.5566 150.6324) (width 0.45) (layer "F.Cu") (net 12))
 (segment (start 217.6272 161.417) (end 217.6272 151.5618) (width 0.45) (layer "F.Cu") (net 12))
 (segment (start 217.1941 162.074737) (end 217.463041 162.074737) (width 0.45) (layer "F.Cu") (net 12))
 (segment (start 217.6272 161.910578) (end 217.6272 161.417) (width 0.45) (layer "F.Cu") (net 12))
 (segment (start 218.5566 150.6324) (end 218.5566 147.2118) (width 0.45) (layer "F.Cu") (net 12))
 (segment (start 217.463041 162.074737) (end 217.6272 161.910578) (width 0.45) (layer "F.Cu") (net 12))
 (via (at 218.5566 146.7358) (size 1.75) (drill 1) (layers "F.Cu" "B.Cu") (free yes) (tenting none) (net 12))
 (via (at 217.6272 156.1592) (size 0.6) (drill 0.3) (layers "F.Cu" "B.Cu") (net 12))
 (via (at 217.6272 161.417) (size 0.6) (drill 0.3) (layers "F.Cu" "B.Cu") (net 12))
 (segment (start 217.6272 156.1592) (end 217.6272 161.417) (width 0.45) (layer "B.Cu") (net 12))
 (segment (start 228.787848 162.009945) (end 228.847393 161.9504) (width 0.45) (layer "F.Cu") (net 10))
 (segment (start 228.93175 161.9504) (end 228.939193 161.942957) (width 0.45) (layer "F.Cu") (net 10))
 (segment (start 228.847393 161.9504) (end 228.93175 161.9504) (width 0.45) (layer "F.Cu") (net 10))
 (segment (start 229.866902 150.472698) (end 229.866902 147.2118) (width 0.45) (layer "F.Cu") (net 10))
 (segment (start 228.939193 161.942957) (end 228.939193 161.3408) (width 0.45) (layer "F.Cu") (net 10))
 (segment (start 228.504402 162.074737) (end 228.569194 162.009945) (width 0.45) (layer "F.Cu") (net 10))
 (segment (start 228.569194 162.009945) (end 228.787848 162.009945) (width 0.45) (layer "F.Cu") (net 10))
 (segment (start 228.939193 161.3408) (end 228.939193 151.400407) (width 0.45) (layer "F.Cu") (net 10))
 (segment (start 228.939193 151.400407) (end 229.866902 150.472698) (width 0.45) (layer "F.Cu") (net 10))
 (segment (start 228.939193 161.3408) (end 228.939193 161.1122) (width 0.45) (layer "F.Cu") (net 10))
 (via (at 229.866902 146.7358) (size 1.75) (drill 1) (layers "F.Cu" "B.Cu") (free yes) (tenting none) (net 10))
 (via (at 228.939193 161.3408) (size 0.6) (drill 0.3) (layers "F.Cu" "B.Cu") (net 10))
 (via (at 228.939193 156.845) (size 0.6) (drill 0.3) (layers "F.Cu" "B.Cu") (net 10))
 (segment (start 228.939193 156.845) (end 228.939193 161.3408) (width 0.45) (layer "B.Cu") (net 10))
 (segment (start 214.4878 160.909) (end 214.9191 161.3403) (width 0.45) (layer "F.Cu") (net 7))
 (segment (start 214.9191 161.3403) (end 214.9191 162.074737) (width 0.45) (layer "F.Cu") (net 7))
 (segment (start 213.3554 154.4828) (end 213.3554 151.892) (width 0.45) (layer "F.Cu") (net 7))
 (segment (start 213.3554 155.6974) (end 213.3554 154.4828) (width 0.45) (layer "F.Cu") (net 7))
 (segment (start 214.4878 156.1846) (end 213.8426 156.1846) (width 0.45) (layer "F.Cu") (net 7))
 (segment (start 214.4878 156.1846) (end 214.4878 160.909) (width 0.45) (layer "F.Cu") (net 7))
 (segment (start 213.8426 156.1846) (end 213.3554 155.6974) (width 0.45) (layer "F.Cu") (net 7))
 (via (at 214.9191 161.3403) (size 0.6) (drill 0.3) (layers "F.Cu" "B.Cu") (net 7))
 (via (at 214.4878 156.1846) (size 0.6) (drill 0.3) (layers "F.Cu" "B.Cu") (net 7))
 (segment (start 214.4878 156.1846) (end 214.4878 160.909) (width 0.45) (layer "B.Cu") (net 7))
 (segment (start 214.4878 160.909) (end 214.9191 161.3403) (width 0.45) (layer "B.Cu") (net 7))
 (segment (start 214.9191 163.024737) (end 215.663863 163.024737) (width 0.45) (layer "F.Cu") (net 5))
 (segment (start 215.577463 163.974737) (end 216.0524 163.4998) (width 0.45) (layer "F.Cu") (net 5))
 (segment (start 214.9191 163.974737) (end 215.577463 163.974737) (width 0.45) (layer "F.Cu") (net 5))
 (segment (start 216.0524 163.4998) (end 216.0524 162.6362) (width 0.45) (layer "F.Cu") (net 5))
 (segment (start 215.9554 151.892) (end 215.9554 154.4828) (width 0.45) (layer "F.Cu") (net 5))
 (segment (start 216.0524 154.5798) (end 215.9554 154.4828) (width 0.45) (layer "F.Cu") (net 5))
 (segment (start 216.0524 156.1846) (end 216.0524 154.5798) (width 0.45) (layer "F.Cu") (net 5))
 (segment (start 216.0524 162.6362) (end 216.0524 161.3916) (width 0.45) (layer "F.Cu") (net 5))
 (segment (start 216.0524 156.1846) (end 216.0524 161.3916) (width 0.45) (layer "F.Cu") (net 5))
 (segment (start 215.663863 163.024737) (end 216.0524 162.6362) (width 0.45) (layer "F.Cu") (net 5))
 (via (at 216.0524 161.3916) (size 0.6) (drill 0.3) (layers "F.Cu" "B.Cu") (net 5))
 (via (at 216.0524 156.1846) (size 0.6) (drill 0.3) (layers "F.Cu" "B.Cu") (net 5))
 (segment (start 216.0524 156.1846) (end 216.0524 161.3916) (width 0.45) (layer "B.Cu") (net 5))
 (segment (start 213.5378 148.7424) (end 213.5378 147.3835) (width 0.45) (layer "F.Cu") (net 8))
 (segment (start 214.6554 151.892) (end 214.6554 150.4442) (width 0.45) (layer "F.Cu") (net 8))
 (segment (start 214.4878 148.7932) (end 213.5886 148.7932) (width 0.45) (layer "F.Cu") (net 8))
 (segment (start 213.5378 149.3266) (end 213.5378 148.7424) (width 0.45) (layer "F.Cu") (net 8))
 (segment (start 213.5886 148.7932) (end 213.5378 148.7424) (width 0.45) (layer "F.Cu") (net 8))
 (segment (start 214.6554 150.4442) (end 213.5378 149.3266) (width 0.45) (layer "F.Cu") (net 8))
 (via (at 213.5566 146.7358) (size 1.75) (drill 1) (layers "F.Cu" "B.Cu") (free yes) (tenting none) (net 8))
 (segment (start 216.0524 147.2118) (end 216.0566 147.2118) (width 0.45) (layer "F.Cu") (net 6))
 (segment (start 216.0778 147.4089) (end 216.0524 147.3835) (width 0.45) (layer "F.Cu") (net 6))
 (segment (start 216.0778 148.7932) (end 216.0778 147.4089) (width 0.45) (layer "F.Cu") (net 6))
 (segment (start 214.6554 154.4828) (end 214.6554 153.289) (width 0.45) (layer "F.Cu") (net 6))
 (segment (start 216.0778 148.7932) (end 215.1278 148.7932) (width 0.45) (layer "F.Cu") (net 6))
 (via (at 216.0778 148.7932) (size 0.6) (drill 0.3) (layers "F.Cu" "B.Cu") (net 6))
 (via (at 214.6554 153.289) (size 0.6) (drill 0.3) (layers "F.Cu" "B.Cu") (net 6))
 (via (at 216.0566 146.7358) (size 1.75) (drill 1) (layers "F.Cu" "B.Cu") (free yes) (tenting none) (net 6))
 (segment (start 216.0778 151.8666) (end 216.0778 148.7932) (width 0.45) (layer "B.Cu") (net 6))
 (segment (start 214.6554 153.289) (end 216.0778 151.8666) (width 0.45) (layer "B.Cu") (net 6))
 (segment (start 226.0346 150.6474) (end 224.8662 149.479) (width 0.45) (layer "F.Cu") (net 2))
 (segment (start 224.8662 149.479) (end 224.8662 148.7424) (width 0.45) (layer "F.Cu") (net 2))
 (segment (start 224.917 148.7932) (end 224.8662 148.7424) (width 0.45) (layer "F.Cu") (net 2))
 (segment (start 226.0346 151.892) (end 226.0346 150.6474) (width 0.45) (layer "F.Cu") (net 2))
 (segment (start 224.8662 148.7424) (end 224.8662 147.3835) (width 0.45) (layer "F.Cu") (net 2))
 (segment (start 225.9878 148.7932) (end 224.917 148.7932) (width 0.45) (layer "F.Cu") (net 2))
 (via (at 224.866902 146.7358) (size 1.75) (drill 1) (layers "F.Cu" "B.Cu") (free yes) (tenting none) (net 2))
 (segment (start 226.0392 153.2428) (end 226.0346 153.2382) (width 0.45) (layer "F.Cu") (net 1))
 (segment (start 226.6532 148.8186) (end 226.6278 148.7932) (width 0.45) (layer "F.Cu") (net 1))
 (segment (start 226.0392 154.4574) (end 226.0392 153.2428) (width 0.45) (layer "F.Cu") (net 1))
 (segment (start 227.4062 148.8186) (end 226.6532 148.8186) (width 0.45) (layer "F.Cu") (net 1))
 (segment (start 227.4062 148.8186) (end 227.4062 147.4089) (width 0.45) (layer "F.Cu") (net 1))
 (segment (start 227.4062 147.4089) (end 227.3808 147.3835) (width 0.45) (layer "F.Cu") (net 1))
 (via (at 226.0346 153.2382) (size 0.6) (drill 0.3) (layers "F.Cu" "B.Cu") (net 1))
 (via (at 227.4062 148.8186) (size 0.6) (drill 0.3) (layers "F.Cu" "B.Cu") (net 1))
 (via (at 227.366902 146.7358) (size 1.75) (drill 1) (layers "F.Cu" "B.Cu") (free yes) (tenting none) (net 1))
 (segment (start 226.0346 153.2382) (end 227.4062 151.8666) (width 0.45) (layer "B.Cu") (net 1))
 (segment (start 227.4062 151.8666) (end 227.4062 148.8186) (width 0.45) (layer "B.Cu") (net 1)))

